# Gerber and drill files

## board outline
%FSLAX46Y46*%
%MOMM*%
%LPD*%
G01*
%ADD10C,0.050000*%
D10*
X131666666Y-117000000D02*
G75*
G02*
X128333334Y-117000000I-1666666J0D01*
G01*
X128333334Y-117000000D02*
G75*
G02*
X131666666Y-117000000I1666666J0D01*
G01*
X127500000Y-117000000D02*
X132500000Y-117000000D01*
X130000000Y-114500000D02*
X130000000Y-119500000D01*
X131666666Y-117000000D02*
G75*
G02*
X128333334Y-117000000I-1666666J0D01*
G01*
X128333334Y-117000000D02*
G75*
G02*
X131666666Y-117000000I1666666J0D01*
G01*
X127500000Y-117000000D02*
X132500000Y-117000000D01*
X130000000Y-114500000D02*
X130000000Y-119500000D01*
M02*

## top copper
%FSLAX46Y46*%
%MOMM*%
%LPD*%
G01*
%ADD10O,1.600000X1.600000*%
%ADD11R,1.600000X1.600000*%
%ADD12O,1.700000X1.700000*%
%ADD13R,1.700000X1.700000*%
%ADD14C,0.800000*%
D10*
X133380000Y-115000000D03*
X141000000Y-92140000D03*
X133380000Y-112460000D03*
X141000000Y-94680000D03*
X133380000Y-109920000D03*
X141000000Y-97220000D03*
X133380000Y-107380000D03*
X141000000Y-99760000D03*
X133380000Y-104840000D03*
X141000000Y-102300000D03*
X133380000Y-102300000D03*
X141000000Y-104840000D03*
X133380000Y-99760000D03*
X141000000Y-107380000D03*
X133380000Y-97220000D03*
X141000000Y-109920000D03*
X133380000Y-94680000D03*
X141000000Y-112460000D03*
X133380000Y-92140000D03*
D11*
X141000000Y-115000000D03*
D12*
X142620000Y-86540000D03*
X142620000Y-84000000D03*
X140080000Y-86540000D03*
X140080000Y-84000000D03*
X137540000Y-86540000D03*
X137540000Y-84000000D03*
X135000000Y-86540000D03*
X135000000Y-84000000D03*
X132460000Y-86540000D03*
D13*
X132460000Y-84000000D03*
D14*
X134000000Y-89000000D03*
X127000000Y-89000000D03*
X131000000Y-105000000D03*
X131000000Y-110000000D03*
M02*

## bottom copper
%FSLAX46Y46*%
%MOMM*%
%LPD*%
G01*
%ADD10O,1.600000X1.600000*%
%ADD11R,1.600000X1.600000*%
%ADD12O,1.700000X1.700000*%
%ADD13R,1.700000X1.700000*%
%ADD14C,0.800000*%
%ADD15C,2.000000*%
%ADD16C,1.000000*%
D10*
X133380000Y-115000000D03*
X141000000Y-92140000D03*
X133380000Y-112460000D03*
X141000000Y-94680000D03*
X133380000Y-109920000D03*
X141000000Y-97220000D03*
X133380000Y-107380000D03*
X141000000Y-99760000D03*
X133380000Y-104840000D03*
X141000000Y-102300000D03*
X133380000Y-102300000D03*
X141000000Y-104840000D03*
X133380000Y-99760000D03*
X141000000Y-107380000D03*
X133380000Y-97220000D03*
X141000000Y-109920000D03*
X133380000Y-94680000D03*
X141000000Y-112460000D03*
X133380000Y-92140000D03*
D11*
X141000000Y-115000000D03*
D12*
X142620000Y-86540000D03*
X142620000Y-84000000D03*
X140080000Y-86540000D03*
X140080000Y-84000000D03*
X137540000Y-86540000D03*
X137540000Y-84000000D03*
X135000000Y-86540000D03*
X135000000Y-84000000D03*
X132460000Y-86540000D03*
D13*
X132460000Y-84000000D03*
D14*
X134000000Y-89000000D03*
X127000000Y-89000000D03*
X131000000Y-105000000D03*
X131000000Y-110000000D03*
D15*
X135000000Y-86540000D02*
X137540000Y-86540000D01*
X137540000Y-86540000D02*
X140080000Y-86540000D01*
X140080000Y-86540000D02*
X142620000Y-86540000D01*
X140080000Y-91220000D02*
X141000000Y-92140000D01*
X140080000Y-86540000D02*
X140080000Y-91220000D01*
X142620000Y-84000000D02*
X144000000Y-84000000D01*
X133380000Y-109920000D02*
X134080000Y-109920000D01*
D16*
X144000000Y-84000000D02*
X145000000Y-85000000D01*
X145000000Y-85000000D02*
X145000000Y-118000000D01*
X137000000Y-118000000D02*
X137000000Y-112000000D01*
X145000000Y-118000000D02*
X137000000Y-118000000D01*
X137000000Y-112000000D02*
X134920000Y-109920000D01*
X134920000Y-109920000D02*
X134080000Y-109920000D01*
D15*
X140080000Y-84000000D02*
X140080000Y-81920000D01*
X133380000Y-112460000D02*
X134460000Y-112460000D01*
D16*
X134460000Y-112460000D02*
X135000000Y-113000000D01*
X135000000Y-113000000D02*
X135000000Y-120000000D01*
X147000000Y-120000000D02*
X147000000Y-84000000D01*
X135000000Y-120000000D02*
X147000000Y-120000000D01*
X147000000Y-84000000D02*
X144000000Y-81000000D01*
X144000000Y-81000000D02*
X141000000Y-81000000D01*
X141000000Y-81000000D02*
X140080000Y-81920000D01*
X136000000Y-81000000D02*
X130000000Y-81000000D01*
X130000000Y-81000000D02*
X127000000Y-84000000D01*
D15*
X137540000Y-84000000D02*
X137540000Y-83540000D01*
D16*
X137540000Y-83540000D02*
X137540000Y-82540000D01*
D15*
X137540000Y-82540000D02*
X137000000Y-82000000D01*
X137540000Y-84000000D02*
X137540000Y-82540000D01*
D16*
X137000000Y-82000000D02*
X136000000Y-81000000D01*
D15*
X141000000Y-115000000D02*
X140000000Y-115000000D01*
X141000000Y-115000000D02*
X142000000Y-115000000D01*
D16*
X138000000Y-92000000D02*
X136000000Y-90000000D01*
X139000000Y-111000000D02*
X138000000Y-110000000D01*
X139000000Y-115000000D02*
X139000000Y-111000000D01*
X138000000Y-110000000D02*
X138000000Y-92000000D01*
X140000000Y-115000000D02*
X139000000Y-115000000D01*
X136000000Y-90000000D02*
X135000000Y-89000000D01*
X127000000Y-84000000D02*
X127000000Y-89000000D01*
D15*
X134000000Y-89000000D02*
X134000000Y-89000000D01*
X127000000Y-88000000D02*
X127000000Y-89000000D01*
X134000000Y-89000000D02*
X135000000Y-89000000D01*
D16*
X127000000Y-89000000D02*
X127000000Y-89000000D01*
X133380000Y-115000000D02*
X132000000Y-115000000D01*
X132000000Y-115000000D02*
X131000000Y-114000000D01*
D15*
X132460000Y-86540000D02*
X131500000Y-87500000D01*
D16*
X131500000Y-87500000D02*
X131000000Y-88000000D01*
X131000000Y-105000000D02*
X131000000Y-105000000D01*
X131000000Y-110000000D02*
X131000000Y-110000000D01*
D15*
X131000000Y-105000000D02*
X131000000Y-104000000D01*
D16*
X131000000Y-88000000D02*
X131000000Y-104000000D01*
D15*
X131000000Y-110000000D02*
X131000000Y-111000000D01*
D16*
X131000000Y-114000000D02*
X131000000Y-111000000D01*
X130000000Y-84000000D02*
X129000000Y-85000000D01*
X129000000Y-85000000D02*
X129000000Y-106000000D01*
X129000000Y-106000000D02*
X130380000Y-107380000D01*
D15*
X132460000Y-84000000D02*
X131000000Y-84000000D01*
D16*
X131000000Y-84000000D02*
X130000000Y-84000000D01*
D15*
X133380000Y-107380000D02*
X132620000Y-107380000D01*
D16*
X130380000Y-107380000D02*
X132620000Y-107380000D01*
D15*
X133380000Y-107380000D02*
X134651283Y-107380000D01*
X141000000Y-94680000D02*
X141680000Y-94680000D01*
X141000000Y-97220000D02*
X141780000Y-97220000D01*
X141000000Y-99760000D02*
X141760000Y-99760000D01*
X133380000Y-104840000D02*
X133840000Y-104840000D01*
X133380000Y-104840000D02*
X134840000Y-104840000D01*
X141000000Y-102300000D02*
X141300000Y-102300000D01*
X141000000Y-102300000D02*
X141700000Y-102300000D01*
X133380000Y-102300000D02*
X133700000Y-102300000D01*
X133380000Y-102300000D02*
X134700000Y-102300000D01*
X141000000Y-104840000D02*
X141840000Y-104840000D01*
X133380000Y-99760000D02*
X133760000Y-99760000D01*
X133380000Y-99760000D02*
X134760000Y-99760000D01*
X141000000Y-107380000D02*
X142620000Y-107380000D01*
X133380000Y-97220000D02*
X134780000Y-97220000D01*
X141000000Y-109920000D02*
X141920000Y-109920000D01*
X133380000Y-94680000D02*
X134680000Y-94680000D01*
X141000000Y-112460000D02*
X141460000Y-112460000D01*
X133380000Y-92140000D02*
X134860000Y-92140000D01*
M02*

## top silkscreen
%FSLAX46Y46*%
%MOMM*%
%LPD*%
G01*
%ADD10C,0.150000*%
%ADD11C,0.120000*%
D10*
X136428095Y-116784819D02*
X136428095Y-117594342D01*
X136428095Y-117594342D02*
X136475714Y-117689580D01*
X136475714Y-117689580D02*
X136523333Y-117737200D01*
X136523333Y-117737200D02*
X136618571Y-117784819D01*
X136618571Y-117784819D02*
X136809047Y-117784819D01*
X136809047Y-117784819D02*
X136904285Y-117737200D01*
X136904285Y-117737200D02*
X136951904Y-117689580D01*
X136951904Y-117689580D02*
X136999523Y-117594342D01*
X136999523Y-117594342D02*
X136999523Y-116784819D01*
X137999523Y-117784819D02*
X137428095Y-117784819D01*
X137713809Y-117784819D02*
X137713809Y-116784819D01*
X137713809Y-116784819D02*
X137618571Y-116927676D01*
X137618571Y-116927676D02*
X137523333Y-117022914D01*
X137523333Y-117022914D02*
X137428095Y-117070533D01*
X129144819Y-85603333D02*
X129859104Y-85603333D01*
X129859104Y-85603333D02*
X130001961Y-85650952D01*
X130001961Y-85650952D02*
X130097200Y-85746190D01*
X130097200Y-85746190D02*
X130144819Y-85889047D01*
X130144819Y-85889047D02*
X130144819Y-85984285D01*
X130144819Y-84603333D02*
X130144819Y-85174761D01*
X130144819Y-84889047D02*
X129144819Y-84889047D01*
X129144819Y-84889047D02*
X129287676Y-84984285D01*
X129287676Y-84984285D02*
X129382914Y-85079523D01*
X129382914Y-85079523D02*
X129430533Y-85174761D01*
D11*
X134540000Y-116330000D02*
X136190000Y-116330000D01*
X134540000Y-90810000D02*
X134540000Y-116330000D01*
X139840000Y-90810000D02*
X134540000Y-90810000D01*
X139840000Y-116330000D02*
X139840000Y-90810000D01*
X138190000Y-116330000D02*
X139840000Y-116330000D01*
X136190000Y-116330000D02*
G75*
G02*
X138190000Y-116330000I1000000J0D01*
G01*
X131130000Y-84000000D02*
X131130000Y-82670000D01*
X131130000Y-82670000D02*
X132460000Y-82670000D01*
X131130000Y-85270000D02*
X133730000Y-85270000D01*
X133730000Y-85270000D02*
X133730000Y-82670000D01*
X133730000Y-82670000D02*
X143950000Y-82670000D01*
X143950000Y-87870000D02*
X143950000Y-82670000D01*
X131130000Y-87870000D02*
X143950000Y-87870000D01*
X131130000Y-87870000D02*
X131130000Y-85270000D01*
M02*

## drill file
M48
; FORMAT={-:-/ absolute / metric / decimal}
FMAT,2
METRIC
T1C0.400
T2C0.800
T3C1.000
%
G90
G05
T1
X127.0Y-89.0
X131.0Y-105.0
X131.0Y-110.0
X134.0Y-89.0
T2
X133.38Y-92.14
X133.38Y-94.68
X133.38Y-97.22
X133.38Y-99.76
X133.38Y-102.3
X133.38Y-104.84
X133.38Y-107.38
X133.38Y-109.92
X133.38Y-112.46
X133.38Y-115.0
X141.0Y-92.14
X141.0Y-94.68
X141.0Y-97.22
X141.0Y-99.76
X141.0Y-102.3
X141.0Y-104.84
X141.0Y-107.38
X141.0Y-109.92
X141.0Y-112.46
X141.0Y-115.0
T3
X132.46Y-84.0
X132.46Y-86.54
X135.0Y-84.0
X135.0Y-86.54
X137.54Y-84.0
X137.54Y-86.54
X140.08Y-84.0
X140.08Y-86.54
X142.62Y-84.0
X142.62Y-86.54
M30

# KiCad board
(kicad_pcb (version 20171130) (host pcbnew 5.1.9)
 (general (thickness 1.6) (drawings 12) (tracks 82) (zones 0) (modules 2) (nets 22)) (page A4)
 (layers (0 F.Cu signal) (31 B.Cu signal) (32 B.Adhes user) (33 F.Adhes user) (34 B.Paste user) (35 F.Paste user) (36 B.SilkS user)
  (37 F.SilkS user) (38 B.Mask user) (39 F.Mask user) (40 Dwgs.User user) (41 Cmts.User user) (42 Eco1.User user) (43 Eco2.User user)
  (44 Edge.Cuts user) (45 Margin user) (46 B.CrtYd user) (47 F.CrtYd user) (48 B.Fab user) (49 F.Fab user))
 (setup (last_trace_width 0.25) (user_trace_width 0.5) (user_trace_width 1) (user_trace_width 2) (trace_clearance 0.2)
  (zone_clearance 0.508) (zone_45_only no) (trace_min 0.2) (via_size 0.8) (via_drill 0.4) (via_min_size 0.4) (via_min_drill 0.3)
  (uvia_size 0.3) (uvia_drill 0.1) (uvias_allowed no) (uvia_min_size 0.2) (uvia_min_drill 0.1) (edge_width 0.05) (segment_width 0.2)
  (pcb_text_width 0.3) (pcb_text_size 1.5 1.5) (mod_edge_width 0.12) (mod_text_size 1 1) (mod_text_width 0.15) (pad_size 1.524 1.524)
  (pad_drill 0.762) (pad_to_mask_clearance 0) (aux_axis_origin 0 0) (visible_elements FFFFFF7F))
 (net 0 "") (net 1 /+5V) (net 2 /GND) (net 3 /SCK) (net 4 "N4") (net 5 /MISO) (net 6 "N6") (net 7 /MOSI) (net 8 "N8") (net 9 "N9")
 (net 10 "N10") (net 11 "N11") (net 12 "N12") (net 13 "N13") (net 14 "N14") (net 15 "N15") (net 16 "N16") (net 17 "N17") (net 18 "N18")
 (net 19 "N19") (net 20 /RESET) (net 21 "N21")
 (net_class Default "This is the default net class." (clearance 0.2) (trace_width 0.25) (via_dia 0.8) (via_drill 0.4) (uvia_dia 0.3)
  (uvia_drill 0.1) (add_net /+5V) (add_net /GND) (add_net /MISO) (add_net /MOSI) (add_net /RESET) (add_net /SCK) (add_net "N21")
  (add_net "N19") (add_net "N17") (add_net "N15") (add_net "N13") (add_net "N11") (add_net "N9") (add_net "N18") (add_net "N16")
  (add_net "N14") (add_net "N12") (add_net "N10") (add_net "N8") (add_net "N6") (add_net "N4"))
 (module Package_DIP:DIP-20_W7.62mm (layer F.Cu) (at 141 115 180)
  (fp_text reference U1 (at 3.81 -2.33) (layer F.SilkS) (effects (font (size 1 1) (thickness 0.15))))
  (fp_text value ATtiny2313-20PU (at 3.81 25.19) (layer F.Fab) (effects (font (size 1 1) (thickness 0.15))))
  (fp_line (start 6.46 -1.33) (end 4.81 -1.33) (layer F.SilkS) (width 0.12))
  (fp_line (start 6.46 24.19) (end 6.46 -1.33) (layer F.SilkS) (width 0.12))
  (fp_line (start 1.16 24.19) (end 6.46 24.19) (layer F.SilkS) (width 0.12))
  (fp_line (start 1.16 -1.33) (end 1.16 24.19) (layer F.SilkS) (width 0.12))
  (fp_line (start 2.81 -1.33) (end 1.16 -1.33) (layer F.SilkS) (width 0.12))
  (fp_arc (start 3.81 -1.33) (end 2.81 -1.33) (angle -180) (layer F.SilkS) (width 0.12))
  (pad 20 thru_hole oval (at 7.62 0 180) (size 1.6 1.6) (drill 0.8) (layers *.Cu *.Mask) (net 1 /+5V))
  (pad 10 thru_hole oval (at 0 22.86 180) (size 1.6 1.6) (drill 0.8) (layers *.Cu *.Mask) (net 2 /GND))
  (pad 19 thru_hole oval (at 7.62 2.54 180) (size 1.6 1.6) (drill 0.8) (layers *.Cu *.Mask) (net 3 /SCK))
  (pad 9 thru_hole oval (at 0 20.32 180) (size 1.6 1.6) (drill 0.8) (layers *.Cu *.Mask) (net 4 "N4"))
  (pad 18 thru_hole oval (at 7.62 5.08 180) (size 1.6 1.6) (drill 0.8) (layers *.Cu *.Mask) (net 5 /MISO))
  (pad 8 thru_hole oval (at 0 17.78 180) (size 1.6 1.6) (drill 0.8) (layers *.Cu *.Mask) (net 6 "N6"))
  (pad 17 thru_hole oval (at 7.62 7.62 180) (size 1.6 1.6) (drill 0.8) (layers *.Cu *.Mask) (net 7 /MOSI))
  (pad 7 thru_hole oval (at 0 15.24 180) (size 1.6 1.6) (drill 0.8) (layers *.Cu *.Mask) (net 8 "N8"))
  (pad 16 thru_hole oval (at 7.62 10.16 180) (size 1.6 1.6) (drill 0.8) (layers *.Cu *.Mask) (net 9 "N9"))
  (pad 6 thru_hole oval (at 0 12.7 180) (size 1.6 1.6) (drill 0.8) (layers *.Cu *.Mask) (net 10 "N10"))
  (pad 15 thru_hole oval (at 7.62 12.7 180) (size 1.6 1.6) (drill 0.8) (layers *.Cu *.Mask) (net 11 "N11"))
  (pad 5 thru_hole oval (at 0 10.16 180) (size 1.6 1.6) (drill 0.8) (layers *.Cu *.Mask) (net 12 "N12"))
  (pad 14 thru_hole oval (at 7.62 15.24 180) (size 1.6 1.6) (drill 0.8) (layers *.Cu *.Mask) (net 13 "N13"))
  (pad 4 thru_hole oval (at 0 7.62 180) (size 1.6 1.6) (drill 0.8) (layers *.Cu *.Mask) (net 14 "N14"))
  (pad 13 thru_hole oval (at 7.62 17.78 180) (size 1.6 1.6) (drill 0.8) (layers *.Cu *.Mask) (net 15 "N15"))
  (pad 3 thru_hole oval (at 0 5.08 180) (size 1.6 1.6) (drill 0.8) (layers *.Cu *.Mask) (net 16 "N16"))
  (pad 12 thru_hole oval (at 7.62 20.32 180) (size 1.6 1.6) (drill 0.8) (layers *.Cu *.Mask) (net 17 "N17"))
  (pad 2 thru_hole oval (at 0 2.54 180) (size 1.6 1.6) (drill 0.8) (layers *.Cu *.Mask) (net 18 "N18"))
  (pad 11 thru_hole oval (at 7.62 22.86 180) (size 1.6 1.6) (drill 0.8) (layers *.Cu *.Mask) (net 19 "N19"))
  (pad 1 thru_hole rect (at 0 0 180) (size 1.6 1.6) (drill 0.8) (layers *.Cu *.Mask) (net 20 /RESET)))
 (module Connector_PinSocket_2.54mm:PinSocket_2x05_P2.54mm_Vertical (layer F.Cu) (at 132.46 84 90)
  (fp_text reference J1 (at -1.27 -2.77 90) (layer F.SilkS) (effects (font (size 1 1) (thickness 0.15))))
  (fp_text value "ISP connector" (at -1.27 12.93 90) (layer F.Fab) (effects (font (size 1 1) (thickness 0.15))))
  (fp_line (start 0 -1.33) (end 1.33 -1.33) (layer F.SilkS) (width 0.12))
  (fp_line (start 1.33 -1.33) (end 1.33 0) (layer F.SilkS) (width 0.12))
  (fp_line (start -1.27 -1.33) (end -1.27 1.27) (layer F.SilkS) (width 0.12))
  (fp_line (start -1.27 1.27) (end 1.33 1.27) (layer F.SilkS) (width 0.12))
  (fp_line (start 1.33 1.27) (end 1.33 11.49) (layer F.SilkS) (width 0.12))
  (fp_line (start -3.87 11.49) (end 1.33 11.49) (layer F.SilkS) (width 0.12))
  (fp_line (start -3.87 -1.33) (end -3.87 11.49) (layer F.SilkS) (width 0.12))
  (fp_line (start -3.87 -1.33) (end -1.27 -1.33) (layer F.SilkS) (width 0.12))
  (pad 10 thru_hole oval (at -2.54 10.16 90) (size 1.7 1.7) (drill 1) (layers *.Cu *.Mask) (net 2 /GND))
  (pad 9 thru_hole oval (at 0 10.16 90) (size 1.7 1.7) (drill 1) (layers *.Cu *.Mask) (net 5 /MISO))
  (pad 8 thru_hole oval (at -2.54 7.62 90) (size 1.7 1.7) (drill 1) (layers *.Cu *.Mask) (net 2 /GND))
  (pad 7 thru_hole oval (at 0 7.62 90) (size 1.7 1.7) (drill 1) (layers *.Cu *.Mask) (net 3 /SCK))
  (pad 6 thru_hole oval (at -2.54 5.08 90) (size 1.7 1.7) (drill 1) (layers *.Cu *.Mask) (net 2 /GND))
  (pad 5 thru_hole oval (at 0 5.08 90) (size 1.7 1.7) (drill 1) (layers *.Cu *.Mask) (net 20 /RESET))
  (pad 4 thru_hole oval (at -2.54 2.54 90) (size 1.7 1.7) (drill 1) (layers *.Cu *.Mask) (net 2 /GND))
  (pad 3 thru_hole oval (at 0 2.54 90) (size 1.7 1.7) (drill 1) (layers *.Cu *.Mask) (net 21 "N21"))
  (pad 2 thru_hole oval (at -2.54 0 90) (size 1.7 1.7) (drill 1) (layers *.Cu *.Mask) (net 1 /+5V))
  (pad 1 thru_hole rect (at 0 0 90) (size 1.7 1.7) (drill 1) (layers *.Cu *.Mask) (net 7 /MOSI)))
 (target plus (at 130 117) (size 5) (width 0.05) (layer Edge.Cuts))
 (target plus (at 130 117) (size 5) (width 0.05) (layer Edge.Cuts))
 (segment (start 135 86.54) (end 137.54 86.54) (width 2) (layer B.Cu) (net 2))
 (segment (start 137.54 86.54) (end 140.08 86.54) (width 2) (layer B.Cu) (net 2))
 (segment (start 140.08 86.54) (end 142.62 86.54) (width 2) (layer B.Cu) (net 2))
 (segment (start 140.08 91.22) (end 141 92.14) (width 2) (layer B.Cu) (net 2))
 (segment (start 140.08 86.54) (end 140.08 91.22) (width 2) (layer B.Cu) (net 2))
 (segment (start 142.62 84) (end 144 84) (width 2) (layer B.Cu) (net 5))
 (segment (start 133.38 109.92) (end 134.08 109.92) (width 2) (layer B.Cu) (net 5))
 (segment (start 144 84) (end 145 85) (width 1) (layer B.Cu) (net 5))
 (segment (start 145 85) (end 145 118) (width 1) (layer B.Cu) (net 5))
 (segment (start 137 118) (end 137 112) (width 1) (layer B.Cu) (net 5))
 (segment (start 145 118) (end 137 118) (width 1) (layer B.Cu) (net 5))
 (segment (start 137 112) (end 134.92 109.92) (width 1) (layer B.Cu) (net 5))
 (segment (start 134.92 109.92) (end 134.08 109.92) (width 1) (layer B.Cu) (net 5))
 (segment (start 140.08 84) (end 140.08 81.92) (width 2) (layer B.Cu) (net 3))
 (segment (start 133.38 112.46) (end 134.46 112.46) (width 2) (layer B.Cu) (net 3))
 (segment (start 134.46 112.46) (end 135 113) (width 1) (layer B.Cu) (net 3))
 (segment (start 135 113) (end 135 120) (width 1) (layer B.Cu) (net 3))
 (segment (start 147 120) (end 147 84) (width 1) (layer B.Cu) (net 3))
 (segment (start 135 120) (end 147 120) (width 1) (layer B.Cu) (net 3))
 (segment (start 147 84) (end 144 81) (width 1) (layer B.Cu) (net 3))
 (segment (start 144 81) (end 141 81) (width 1) (layer B.Cu) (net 3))
 (segment (start 141 81) (end 140.08 81.92) (width 1) (layer B.Cu) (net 3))
 (segment (start 136 81) (end 130 81) (width 1) (layer B.Cu) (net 20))
 (segment (start 130 81) (end 127 84) (width 1) (layer B.Cu) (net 20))
 (segment (start 137.54 84) (end 137.54 83.54) (width 2) (layer B.Cu) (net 20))
 (segment (start 137.54 83.54) (end 137.54 82.54) (width 1) (layer B.Cu) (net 20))
 (segment (start 137.54 82.54) (end 137 82) (width 2) (layer B.Cu) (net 20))
 (segment (start 137.54 84) (end 137.54 82.54) (width 2) (layer B.Cu) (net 20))
 (segment (start 137 82) (end 136 81) (width 1) (layer B.Cu) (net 20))
 (segment (start 141 115) (end 140 115) (width 2) (layer B.Cu) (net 20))
 (segment (start 141 115) (end 142 115) (width 2) (layer B.Cu) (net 20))
 (segment (start 138 92) (end 136 90) (width 1) (layer B.Cu) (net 20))
 (segment (start 139 111) (end 138 110) (width 1) (layer B.Cu) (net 20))
 (segment (start 139 115) (end 139 111) (width 1) (layer B.Cu) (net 20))
 (segment (start 138 110) (end 138 92) (width 1) (layer B.Cu) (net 20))
 (segment (start 140 115) (end 139 115) (width 1) (layer B.Cu) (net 20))
 (segment (start 136 90) (end 135 89) (width 1) (layer B.Cu) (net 20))
 (segment (start 127 84) (end 127 89) (width 1) (layer B.Cu) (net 20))
 (segment (start 134 89) (end 134 89) (width 2) (layer B.Cu) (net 20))
 (segment (start 127 88) (end 127 89) (width 2) (layer B.Cu) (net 20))
 (segment (start 134 89) (end 135 89) (width 2) (layer B.Cu) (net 20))
 (via (at 134 89) (size 0.8) (drill 0.4) (layers F.Cu B.Cu) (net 20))
 (segment (start 127 89) (end 127 89) (width 1) (layer B.Cu) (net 20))
 (via (at 127 89) (size 0.8) (drill 0.4) (layers F.Cu B.Cu) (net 20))
 (segment (start 133.38 115) (end 132 115) (width 1) (layer B.Cu) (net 1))
 (segment (start 132 115) (end 131 114) (width 1) (layer B.Cu) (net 1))
 (segment (start 132.46 86.54) (end 131.5 87.5) (width 2) (layer B.Cu) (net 1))
 (segment (start 131.5 87.5) (end 131 88) (width 1) (layer B.Cu) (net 1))
 (segment (start 131 105) (end 131 105) (width 1) (layer B.Cu) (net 1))
 (via (at 131 105) (size 0.8) (drill 0.4) (layers F.Cu B.Cu) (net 1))
 (segment (start 131 110) (end 131 110) (width 1) (layer B.Cu) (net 1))
 (via (at 131 110) (size 0.8) (drill 0.4) (layers F.Cu B.Cu) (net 1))
 (segment (start 131 105) (end 131 104) (width 2) (layer B.Cu) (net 1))
 (segment (start 131 88) (end 131 104) (width 1) (layer B.Cu) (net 1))
 (segment (start 131 110) (end 131 111) (width 2) (layer B.Cu) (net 1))
 (segment (start 131 114) (end 131 111) (width 1) (layer B.Cu) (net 1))
 (segment (start 130 84) (end 129 85) (width 1) (layer B.Cu) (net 7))
 (segment (start 129 85) (end 129 106) (width 1) (layer B.Cu) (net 7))
 (segment (start 129 106) (end 130.38 107.38) (width 1) (layer B.Cu) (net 7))
 (segment (start 132.46 84) (end 131 84) (width 2) (layer B.Cu) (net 7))
 (segment (start 131 84) (end 130 84) (width 1) (layer B.Cu) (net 7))
 (segment (start 133.38 107.38) (end 132.62 107.38) (width 2) (layer B.Cu) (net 7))
 (segment (start 130.38 107.38) (end 132.62 107.38) (width 1) (layer B.Cu) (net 7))
 (segment (start 133.38 107.38) (end 134.651283 107.38) (width 2) (layer B.Cu) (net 7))
 (segment (start 141 94.68) (end 141.68 94.68) (width 2) (layer B.Cu) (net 4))
 (segment (start 141 97.22) (end 141.78 97.22) (width 2) (layer B.Cu) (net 6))
 (segment (start 141 99.76) (end 141.76 99.76) (width 2) (layer B.Cu) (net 8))
 (segment (start 133.38 104.84) (end 133.84 104.84) (width 2) (layer B.Cu) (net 9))
 (segment (start 133.38 104.84) (end 134.84 104.84) (width 2) (layer B.Cu) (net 9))
 (segment (start 141 102.3) (end 141.3 102.3) (width 2) (layer B.Cu) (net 10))
 (segment (start 141 102.3) (end 141.7 102.3) (width 2) (layer B.Cu) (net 10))
 (segment (start 133.38 102.3) (end 133.7 102.3) (width 2) (layer B.Cu) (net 11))
 (segment (start 133.38 102.3) (end 134.7 102.3) (width 2) (layer B.Cu) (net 11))
 (segment (start 141 104.84) (end 141.84 104.84) (width 2) (layer B.Cu) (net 12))
 (segment (start 133.38 99.76) (end 133.76 99.76) (width 2) (layer B.Cu) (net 13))
 (segment (start 133.38 99.76) (end 134.76 99.76) (width 2) (layer B.Cu) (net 13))
 (segment (start 141 107.38) (end 142.62 107.38) (width 2) (layer B.Cu) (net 14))
 (segment (start 133.38 97.22) (end 134.78 97.22) (width 2) (layer B.Cu) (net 15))
 (segment (start 141 109.92) (end 141.92 109.92) (width 2) (layer B.Cu) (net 16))
 (segment (start 133.38 94.68) (end 134.68 94.68) (width 2) (layer B.Cu) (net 17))
 (segment (start 141 112.46) (end 141.46 112.46) (width 2) (layer B.Cu) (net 18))
 (segment (start 133.38 92.14) (end 134.86 92.14) (width 2) (layer B.Cu) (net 19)))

